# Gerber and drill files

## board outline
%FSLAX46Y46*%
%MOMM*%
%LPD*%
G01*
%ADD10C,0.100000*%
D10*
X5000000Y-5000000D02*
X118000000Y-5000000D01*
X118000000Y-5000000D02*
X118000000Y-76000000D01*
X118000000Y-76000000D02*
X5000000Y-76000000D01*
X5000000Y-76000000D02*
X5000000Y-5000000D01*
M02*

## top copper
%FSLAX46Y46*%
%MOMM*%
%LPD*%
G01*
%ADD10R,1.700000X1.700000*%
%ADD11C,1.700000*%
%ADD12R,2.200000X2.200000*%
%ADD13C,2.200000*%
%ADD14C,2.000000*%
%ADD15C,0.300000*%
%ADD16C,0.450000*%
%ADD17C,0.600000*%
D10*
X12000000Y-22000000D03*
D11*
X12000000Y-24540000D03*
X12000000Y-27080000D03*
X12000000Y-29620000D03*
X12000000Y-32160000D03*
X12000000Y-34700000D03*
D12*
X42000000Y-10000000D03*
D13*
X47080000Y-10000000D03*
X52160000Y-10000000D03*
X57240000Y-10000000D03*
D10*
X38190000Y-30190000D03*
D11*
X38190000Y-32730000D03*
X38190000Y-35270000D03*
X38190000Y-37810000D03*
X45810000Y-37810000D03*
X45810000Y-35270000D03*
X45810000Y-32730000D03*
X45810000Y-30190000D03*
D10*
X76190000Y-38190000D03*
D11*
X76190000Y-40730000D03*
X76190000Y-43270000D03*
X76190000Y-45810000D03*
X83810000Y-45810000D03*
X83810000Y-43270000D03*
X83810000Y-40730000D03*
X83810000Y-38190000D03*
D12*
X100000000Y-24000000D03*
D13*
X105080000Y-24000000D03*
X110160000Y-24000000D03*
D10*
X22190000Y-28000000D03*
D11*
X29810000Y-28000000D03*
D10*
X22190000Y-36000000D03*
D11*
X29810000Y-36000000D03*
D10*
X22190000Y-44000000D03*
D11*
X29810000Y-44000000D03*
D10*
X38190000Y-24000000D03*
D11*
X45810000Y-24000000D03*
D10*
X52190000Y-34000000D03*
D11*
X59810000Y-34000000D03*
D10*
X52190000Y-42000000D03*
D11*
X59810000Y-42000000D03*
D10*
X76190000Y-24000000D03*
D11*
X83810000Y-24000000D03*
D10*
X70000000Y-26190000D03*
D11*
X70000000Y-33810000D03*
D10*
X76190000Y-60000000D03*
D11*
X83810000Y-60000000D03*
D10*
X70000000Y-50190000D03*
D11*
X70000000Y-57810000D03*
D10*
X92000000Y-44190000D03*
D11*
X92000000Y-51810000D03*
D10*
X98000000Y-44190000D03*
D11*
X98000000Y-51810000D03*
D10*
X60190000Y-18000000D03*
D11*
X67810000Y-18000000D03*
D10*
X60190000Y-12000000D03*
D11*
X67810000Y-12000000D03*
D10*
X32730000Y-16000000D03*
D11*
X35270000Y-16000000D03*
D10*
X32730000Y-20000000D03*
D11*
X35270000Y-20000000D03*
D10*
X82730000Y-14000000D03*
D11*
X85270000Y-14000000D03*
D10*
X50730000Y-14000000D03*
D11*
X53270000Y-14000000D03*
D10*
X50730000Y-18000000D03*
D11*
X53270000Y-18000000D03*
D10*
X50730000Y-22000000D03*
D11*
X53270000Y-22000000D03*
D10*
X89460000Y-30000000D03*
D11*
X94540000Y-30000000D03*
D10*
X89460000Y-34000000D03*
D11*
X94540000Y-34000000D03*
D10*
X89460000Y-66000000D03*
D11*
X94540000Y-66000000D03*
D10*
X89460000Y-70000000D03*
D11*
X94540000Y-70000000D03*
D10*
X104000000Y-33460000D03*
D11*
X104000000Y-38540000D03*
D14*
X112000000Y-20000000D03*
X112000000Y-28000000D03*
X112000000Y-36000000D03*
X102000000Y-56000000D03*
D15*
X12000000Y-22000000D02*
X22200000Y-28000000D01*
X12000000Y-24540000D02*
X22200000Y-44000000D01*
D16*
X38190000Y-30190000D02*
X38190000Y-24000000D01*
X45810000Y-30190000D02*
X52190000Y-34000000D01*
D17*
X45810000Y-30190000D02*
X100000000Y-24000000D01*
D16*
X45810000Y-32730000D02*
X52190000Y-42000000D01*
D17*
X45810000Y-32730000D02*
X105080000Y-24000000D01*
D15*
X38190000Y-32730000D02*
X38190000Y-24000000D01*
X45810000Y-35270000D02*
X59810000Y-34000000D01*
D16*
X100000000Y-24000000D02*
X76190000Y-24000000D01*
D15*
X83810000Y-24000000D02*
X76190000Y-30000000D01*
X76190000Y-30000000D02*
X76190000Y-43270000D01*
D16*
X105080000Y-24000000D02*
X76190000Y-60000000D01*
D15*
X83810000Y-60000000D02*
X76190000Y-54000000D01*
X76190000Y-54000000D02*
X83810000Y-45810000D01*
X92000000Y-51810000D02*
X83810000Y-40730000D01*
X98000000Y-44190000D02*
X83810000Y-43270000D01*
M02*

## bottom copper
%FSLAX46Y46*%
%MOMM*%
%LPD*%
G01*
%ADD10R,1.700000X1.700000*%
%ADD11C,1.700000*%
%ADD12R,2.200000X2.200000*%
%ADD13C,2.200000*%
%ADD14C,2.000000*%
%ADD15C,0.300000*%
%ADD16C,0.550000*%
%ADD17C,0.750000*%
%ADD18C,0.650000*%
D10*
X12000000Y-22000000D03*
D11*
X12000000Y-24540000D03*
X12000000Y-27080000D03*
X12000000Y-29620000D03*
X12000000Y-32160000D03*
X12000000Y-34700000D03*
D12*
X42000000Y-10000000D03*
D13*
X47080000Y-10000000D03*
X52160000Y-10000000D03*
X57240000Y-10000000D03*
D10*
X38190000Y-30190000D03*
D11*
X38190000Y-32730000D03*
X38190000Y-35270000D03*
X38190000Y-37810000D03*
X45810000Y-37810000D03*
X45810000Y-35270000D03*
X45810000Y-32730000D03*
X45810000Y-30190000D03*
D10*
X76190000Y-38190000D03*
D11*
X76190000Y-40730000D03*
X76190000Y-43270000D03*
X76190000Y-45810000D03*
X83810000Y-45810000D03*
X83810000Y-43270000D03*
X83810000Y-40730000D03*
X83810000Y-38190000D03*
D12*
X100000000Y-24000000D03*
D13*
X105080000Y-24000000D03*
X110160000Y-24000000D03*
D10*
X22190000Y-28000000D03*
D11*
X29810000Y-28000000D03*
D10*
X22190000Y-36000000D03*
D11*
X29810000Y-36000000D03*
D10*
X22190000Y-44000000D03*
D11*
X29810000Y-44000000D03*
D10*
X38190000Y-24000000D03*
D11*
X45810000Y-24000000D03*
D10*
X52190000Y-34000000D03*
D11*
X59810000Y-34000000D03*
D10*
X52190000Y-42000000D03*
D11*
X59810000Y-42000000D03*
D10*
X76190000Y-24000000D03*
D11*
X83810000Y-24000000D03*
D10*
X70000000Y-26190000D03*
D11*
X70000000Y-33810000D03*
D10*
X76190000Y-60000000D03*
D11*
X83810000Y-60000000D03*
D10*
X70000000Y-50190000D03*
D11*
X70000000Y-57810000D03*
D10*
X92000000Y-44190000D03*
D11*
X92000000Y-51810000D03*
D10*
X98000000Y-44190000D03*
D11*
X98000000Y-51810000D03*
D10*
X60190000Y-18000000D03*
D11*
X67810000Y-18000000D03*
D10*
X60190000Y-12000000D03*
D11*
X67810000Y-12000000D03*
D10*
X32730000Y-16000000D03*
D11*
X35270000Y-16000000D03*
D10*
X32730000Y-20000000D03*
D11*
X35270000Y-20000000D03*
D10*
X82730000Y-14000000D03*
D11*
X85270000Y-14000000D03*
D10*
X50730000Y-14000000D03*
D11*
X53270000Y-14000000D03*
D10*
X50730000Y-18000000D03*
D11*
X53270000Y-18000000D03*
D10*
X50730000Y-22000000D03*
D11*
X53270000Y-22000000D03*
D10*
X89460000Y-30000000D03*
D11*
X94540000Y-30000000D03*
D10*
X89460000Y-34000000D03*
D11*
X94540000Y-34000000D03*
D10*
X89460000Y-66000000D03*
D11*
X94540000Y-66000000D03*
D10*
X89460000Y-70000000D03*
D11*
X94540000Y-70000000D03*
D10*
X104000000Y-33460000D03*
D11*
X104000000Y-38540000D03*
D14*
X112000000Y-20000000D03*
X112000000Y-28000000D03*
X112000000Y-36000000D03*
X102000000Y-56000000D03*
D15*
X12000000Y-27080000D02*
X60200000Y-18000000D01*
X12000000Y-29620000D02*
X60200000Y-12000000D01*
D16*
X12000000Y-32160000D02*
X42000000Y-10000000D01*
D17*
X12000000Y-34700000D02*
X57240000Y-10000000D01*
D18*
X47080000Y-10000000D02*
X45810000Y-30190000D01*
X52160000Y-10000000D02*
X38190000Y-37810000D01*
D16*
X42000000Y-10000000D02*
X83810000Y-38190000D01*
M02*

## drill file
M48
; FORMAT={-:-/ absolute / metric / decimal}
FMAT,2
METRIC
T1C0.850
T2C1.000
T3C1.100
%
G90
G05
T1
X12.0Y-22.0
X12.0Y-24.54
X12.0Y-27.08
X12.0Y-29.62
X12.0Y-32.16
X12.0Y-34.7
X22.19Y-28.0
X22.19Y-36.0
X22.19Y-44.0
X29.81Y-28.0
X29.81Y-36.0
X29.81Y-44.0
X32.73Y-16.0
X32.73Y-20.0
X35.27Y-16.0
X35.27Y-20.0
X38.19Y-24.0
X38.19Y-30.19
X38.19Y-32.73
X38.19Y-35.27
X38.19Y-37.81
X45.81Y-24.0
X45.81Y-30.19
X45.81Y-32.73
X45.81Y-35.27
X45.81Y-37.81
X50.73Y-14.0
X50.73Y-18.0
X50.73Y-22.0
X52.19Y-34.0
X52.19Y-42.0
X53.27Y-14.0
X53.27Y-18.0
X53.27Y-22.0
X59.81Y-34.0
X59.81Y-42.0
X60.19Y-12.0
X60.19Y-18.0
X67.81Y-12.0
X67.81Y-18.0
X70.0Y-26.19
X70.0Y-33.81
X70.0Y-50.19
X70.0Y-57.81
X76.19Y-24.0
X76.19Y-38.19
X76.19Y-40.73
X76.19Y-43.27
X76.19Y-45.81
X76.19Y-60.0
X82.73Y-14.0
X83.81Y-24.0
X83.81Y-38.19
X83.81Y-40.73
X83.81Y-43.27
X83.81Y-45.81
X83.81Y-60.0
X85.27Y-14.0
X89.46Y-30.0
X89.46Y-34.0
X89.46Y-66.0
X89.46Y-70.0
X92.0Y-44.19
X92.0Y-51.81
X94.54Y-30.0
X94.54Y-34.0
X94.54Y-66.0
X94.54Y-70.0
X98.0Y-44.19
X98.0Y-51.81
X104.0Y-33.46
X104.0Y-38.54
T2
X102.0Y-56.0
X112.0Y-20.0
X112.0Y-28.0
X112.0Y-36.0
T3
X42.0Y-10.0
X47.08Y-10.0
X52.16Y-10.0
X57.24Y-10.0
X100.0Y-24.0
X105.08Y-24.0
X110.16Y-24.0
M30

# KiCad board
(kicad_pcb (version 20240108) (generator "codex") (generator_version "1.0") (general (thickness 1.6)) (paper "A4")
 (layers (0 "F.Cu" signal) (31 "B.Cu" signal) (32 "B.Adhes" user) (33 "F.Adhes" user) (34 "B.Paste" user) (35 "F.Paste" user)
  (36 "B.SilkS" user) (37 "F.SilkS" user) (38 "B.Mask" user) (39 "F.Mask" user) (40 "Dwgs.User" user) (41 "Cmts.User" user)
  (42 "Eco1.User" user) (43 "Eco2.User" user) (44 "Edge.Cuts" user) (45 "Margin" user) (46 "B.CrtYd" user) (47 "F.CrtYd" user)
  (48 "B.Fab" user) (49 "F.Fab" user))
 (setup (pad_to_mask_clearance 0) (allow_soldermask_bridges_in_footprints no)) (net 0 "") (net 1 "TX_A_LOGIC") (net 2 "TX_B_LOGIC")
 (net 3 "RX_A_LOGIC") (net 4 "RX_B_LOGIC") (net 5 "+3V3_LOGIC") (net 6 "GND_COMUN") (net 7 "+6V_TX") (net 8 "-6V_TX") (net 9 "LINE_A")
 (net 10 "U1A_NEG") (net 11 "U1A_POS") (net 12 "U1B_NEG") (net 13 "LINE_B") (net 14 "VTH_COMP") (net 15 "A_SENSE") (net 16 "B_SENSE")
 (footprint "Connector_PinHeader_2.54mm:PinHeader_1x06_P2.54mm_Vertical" (layer "F.Cu") (at 12.00 22.00)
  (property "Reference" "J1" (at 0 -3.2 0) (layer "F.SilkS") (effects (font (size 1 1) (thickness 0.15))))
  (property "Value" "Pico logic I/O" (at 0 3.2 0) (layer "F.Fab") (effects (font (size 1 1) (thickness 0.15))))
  (pad "1" thru_hole rect (at 0.00 0.00) (size 1.70 1.70) (drill 0.85) (layers "*.Cu" "*.Mask") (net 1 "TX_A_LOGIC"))
  (pad "2" thru_hole circle (at 0.00 2.54) (size 1.70 1.70) (drill 0.85) (layers "*.Cu" "*.Mask") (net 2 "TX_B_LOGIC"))
  (pad "3" thru_hole circle (at 0.00 5.08) (size 1.70 1.70) (drill 0.85) (layers "*.Cu" "*.Mask") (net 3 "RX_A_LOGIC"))
  (pad "4" thru_hole circle (at 0.00 7.62) (size 1.70 1.70) (drill 0.85) (layers "*.Cu" "*.Mask") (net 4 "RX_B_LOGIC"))
  (pad "5" thru_hole circle (at 0.00 10.16) (size 1.70 1.70) (drill 0.85) (layers "*.Cu" "*.Mask") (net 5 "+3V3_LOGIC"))
  (pad "6" thru_hole circle (at 0.00 12.70) (size 1.70 1.70) (drill 0.85) (layers "*.Cu" "*.Mask") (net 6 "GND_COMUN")))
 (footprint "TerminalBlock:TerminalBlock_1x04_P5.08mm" (layer "F.Cu") (at 42.00 10.00)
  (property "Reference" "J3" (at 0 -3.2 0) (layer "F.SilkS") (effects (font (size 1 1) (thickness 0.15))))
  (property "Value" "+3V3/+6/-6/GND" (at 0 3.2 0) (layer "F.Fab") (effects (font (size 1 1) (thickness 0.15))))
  (pad "1" thru_hole rect (at 0.00 0.00) (size 2.20 2.20) (drill 1.10) (layers "*.Cu" "*.Mask") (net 5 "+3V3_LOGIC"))
  (pad "2" thru_hole circle (at 5.08 0.00) (size 2.20 2.20) (drill 1.10) (layers "*.Cu" "*.Mask") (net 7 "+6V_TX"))
  (pad "3" thru_hole circle (at 10.16 0.00) (size 2.20 2.20) (drill 1.10) (layers "*.Cu" "*.Mask") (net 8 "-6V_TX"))
  (pad "4" thru_hole circle (at 15.24 0.00) (size 2.20 2.20) (drill 1.10) (layers "*.Cu" "*.Mask") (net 6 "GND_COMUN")))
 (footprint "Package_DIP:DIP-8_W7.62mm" (layer "F.Cu") (at 42.00 34.00)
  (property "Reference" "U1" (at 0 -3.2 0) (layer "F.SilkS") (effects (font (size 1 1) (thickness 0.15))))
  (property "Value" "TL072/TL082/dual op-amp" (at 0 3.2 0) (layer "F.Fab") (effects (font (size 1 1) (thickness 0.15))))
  (pad "1" thru_hole rect (at -3.81 -3.81) (size 1.70 1.70) (drill 0.85) (layers "*.Cu" "*.Mask") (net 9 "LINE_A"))
  (pad "2" thru_hole circle (at -3.81 -1.27) (size 1.70 1.70) (drill 0.85) (layers "*.Cu" "*.Mask") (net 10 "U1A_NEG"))
  (pad "3" thru_hole circle (at -3.81 1.27) (size 1.70 1.70) (drill 0.85) (layers "*.Cu" "*.Mask") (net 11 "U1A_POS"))
  (pad "4" thru_hole circle (at -3.81 3.81) (size 1.70 1.70) (drill 0.85) (layers "*.Cu" "*.Mask") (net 8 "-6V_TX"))
  (pad "5" thru_hole circle (at 3.81 3.81) (size 1.70 1.70) (drill 0.85) (layers "*.Cu" "*.Mask") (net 6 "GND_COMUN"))
  (pad "6" thru_hole circle (at 3.81 1.27) (size 1.70 1.70) (drill 0.85) (layers "*.Cu" "*.Mask") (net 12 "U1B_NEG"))
  (pad "7" thru_hole circle (at 3.81 -1.27) (size 1.70 1.70) (drill 0.85) (layers "*.Cu" "*.Mask") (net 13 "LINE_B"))
  (pad "8" thru_hole circle (at 3.81 -3.81) (size 1.70 1.70) (drill 0.85) (layers "*.Cu" "*.Mask") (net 7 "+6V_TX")))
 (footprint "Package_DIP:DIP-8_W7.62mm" (layer "F.Cu") (at 80.00 42.00)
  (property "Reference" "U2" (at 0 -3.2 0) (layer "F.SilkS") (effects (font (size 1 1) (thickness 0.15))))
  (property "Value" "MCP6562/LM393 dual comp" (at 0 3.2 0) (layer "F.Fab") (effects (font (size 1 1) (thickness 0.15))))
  (pad "1" thru_hole rect (at -3.81 -3.81) (size 1.70 1.70) (drill 0.85) (layers "*.Cu" "*.Mask") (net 3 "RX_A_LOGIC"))
  (pad "2" thru_hole circle (at -3.81 -1.27) (size 1.70 1.70) (drill 0.85) (layers "*.Cu" "*.Mask") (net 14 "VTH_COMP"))
  (pad "3" thru_hole circle (at -3.81 1.27) (size 1.70 1.70) (drill 0.85) (layers "*.Cu" "*.Mask") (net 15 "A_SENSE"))
  (pad "4" thru_hole circle (at -3.81 3.81) (size 1.70 1.70) (drill 0.85) (layers "*.Cu" "*.Mask") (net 6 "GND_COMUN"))
  (pad "5" thru_hole circle (at 3.81 3.81) (size 1.70 1.70) (drill 0.85) (layers "*.Cu" "*.Mask") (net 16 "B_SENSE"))
  (pad "6" thru_hole circle (at 3.81 1.27) (size 1.70 1.70) (drill 0.85) (layers "*.Cu" "*.Mask") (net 14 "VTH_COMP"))
  (pad "7" thru_hole circle (at 3.81 -1.27) (size 1.70 1.70) (drill 0.85) (layers "*.Cu" "*.Mask") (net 4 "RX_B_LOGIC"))
  (pad "8" thru_hole circle (at 3.81 -3.81) (size 1.70 1.70) (drill 0.85) (layers "*.Cu" "*.Mask") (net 5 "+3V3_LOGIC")))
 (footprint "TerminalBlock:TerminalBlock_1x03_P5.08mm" (layer "F.Cu") (at 100.00 24.00)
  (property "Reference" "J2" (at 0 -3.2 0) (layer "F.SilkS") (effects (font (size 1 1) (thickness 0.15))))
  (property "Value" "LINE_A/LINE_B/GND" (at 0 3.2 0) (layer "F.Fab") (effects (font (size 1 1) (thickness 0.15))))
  (pad "1" thru_hole rect (at 0.00 0.00) (size 2.20 2.20) (drill 1.10) (layers "*.Cu" "*.Mask") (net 9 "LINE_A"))
  (pad "2" thru_hole circle (at 5.08 0.00) (size 2.20 2.20) (drill 1.10) (layers "*.Cu" "*.Mask") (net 13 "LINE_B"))
  (pad "3" thru_hole circle (at 10.16 0.00) (size 2.20 2.20) (drill 1.10) (layers "*.Cu" "*.Mask") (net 6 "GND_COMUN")))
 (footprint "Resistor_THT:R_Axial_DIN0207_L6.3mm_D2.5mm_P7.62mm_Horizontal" (layer "F.Cu") (at 26.00 28.00)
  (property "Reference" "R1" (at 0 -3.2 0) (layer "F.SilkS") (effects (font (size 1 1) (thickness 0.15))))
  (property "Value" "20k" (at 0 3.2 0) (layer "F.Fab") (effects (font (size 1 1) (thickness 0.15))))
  (pad "1" thru_hole rect (at -3.81 0.00) (size 1.70 1.70) (drill 0.85) (layers "*.Cu" "*.Mask") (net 1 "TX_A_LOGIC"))
  (pad "2" thru_hole circle (at 3.81 0.00) (size 1.70 1.70) (drill 0.85) (layers "*.Cu" "*.Mask") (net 11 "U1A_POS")))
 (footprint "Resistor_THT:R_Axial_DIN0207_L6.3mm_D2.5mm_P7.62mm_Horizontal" (layer "F.Cu") (at 26.00 36.00)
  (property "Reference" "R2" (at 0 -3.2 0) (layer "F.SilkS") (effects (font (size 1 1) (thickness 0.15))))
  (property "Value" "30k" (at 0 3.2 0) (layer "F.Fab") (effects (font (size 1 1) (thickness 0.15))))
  (pad "1" thru_hole rect (at -3.81 0.00) (size 1.70 1.70) (drill 0.85) (layers "*.Cu" "*.Mask") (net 11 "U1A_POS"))
  (pad "2" thru_hole circle (at 3.81 0.00) (size 1.70 1.70) (drill 0.85) (layers "*.Cu" "*.Mask") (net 6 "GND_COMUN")))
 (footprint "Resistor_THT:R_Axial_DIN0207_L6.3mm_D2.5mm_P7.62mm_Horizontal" (layer "F.Cu") (at 26.00 44.00)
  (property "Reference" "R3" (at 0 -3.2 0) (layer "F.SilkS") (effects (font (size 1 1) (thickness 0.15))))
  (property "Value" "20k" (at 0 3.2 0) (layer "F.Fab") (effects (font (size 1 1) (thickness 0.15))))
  (pad "1" thru_hole rect (at -3.81 0.00) (size 1.70 1.70) (drill 0.85) (layers "*.Cu" "*.Mask") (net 2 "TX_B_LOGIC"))
  (pad "2" thru_hole circle (at 3.81 0.00) (size 1.70 1.70) (drill 0.85) (layers "*.Cu" "*.Mask") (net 10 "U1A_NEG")))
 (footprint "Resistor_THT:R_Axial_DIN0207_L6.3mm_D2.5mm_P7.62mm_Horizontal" (layer "F.Cu") (at 42.00 24.00)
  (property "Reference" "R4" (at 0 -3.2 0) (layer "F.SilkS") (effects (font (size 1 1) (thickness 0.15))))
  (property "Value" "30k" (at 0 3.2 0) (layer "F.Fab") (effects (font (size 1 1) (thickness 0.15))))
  (pad "1" thru_hole rect (at -3.81 0.00) (size 1.70 1.70) (drill 0.85) (layers "*.Cu" "*.Mask") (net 9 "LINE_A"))
  (pad "2" thru_hole circle (at 3.81 0.00) (size 1.70 1.70) (drill 0.85) (layers "*.Cu" "*.Mask") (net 10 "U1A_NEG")))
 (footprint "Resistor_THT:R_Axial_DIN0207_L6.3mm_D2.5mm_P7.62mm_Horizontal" (layer "F.Cu") (at 56.00 34.00)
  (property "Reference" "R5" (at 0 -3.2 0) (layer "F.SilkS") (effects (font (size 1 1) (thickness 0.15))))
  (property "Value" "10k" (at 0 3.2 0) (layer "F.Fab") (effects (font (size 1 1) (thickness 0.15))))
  (pad "1" thru_hole rect (at -3.81 0.00) (size 1.70 1.70) (drill 0.85) (layers "*.Cu" "*.Mask") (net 9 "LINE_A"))
  (pad "2" thru_hole circle (at 3.81 0.00) (size 1.70 1.70) (drill 0.85) (layers "*.Cu" "*.Mask") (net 12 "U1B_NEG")))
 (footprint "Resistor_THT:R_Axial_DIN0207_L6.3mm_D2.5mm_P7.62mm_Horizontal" (layer "F.Cu") (at 56.00 42.00)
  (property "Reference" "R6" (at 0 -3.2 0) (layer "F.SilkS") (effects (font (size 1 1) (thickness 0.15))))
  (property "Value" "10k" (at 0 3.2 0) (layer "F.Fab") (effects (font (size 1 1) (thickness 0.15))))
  (pad "1" thru_hole rect (at -3.81 0.00) (size 1.70 1.70) (drill 0.85) (layers "*.Cu" "*.Mask") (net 13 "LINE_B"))
  (pad "2" thru_hole circle (at 3.81 0.00) (size 1.70 1.70) (drill 0.85) (layers "*.Cu" "*.Mask") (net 12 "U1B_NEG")))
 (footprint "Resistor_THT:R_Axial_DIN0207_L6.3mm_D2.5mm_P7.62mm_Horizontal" (layer "F.Cu") (at 80.00 24.00)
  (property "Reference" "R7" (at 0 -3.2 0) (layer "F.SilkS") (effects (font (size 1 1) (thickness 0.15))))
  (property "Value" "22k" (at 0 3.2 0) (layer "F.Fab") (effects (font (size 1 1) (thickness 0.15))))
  (pad "1" thru_hole rect (at -3.81 0.00) (size 1.70 1.70) (drill 0.85) (layers "*.Cu" "*.Mask") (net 9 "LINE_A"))
  (pad "2" thru_hole circle (at 3.81 0.00) (size 1.70 1.70) (drill 0.85) (layers "*.Cu" "*.Mask") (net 15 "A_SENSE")))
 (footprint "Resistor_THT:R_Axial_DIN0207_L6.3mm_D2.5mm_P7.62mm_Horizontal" (layer "F.Cu") (at 70.00 30.00)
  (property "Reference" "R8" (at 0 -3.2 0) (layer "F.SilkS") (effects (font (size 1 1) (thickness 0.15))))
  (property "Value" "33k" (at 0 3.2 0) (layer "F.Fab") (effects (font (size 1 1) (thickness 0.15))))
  (pad "1" thru_hole rect (at 0.00 -3.81) (size 1.70 1.70) (drill 0.85) (layers "*.Cu" "*.Mask") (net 15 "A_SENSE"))
  (pad "2" thru_hole circle (at 0.00 3.81) (size 1.70 1.70) (drill 0.85) (layers "*.Cu" "*.Mask") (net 6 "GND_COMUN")))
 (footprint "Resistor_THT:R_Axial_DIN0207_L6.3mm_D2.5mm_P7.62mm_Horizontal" (layer "F.Cu") (at 80.00 60.00)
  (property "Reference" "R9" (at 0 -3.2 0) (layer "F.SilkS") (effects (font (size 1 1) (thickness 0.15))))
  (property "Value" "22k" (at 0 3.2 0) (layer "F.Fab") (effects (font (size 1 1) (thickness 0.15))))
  (pad "1" thru_hole rect (at -3.81 0.00) (size 1.70 1.70) (drill 0.85) (layers "*.Cu" "*.Mask") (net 13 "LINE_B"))
  (pad "2" thru_hole circle (at 3.81 0.00) (size 1.70 1.70) (drill 0.85) (layers "*.Cu" "*.Mask") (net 16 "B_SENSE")))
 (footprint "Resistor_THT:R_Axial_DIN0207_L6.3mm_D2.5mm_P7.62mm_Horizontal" (layer "F.Cu") (at 70.00 54.00)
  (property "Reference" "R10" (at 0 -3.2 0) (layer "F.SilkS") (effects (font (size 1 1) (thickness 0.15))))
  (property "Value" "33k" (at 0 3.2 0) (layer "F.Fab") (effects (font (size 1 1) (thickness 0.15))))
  (pad "1" thru_hole rect (at 0.00 -3.81) (size 1.70 1.70) (drill 0.85) (layers "*.Cu" "*.Mask") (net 16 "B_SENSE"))
  (pad "2" thru_hole circle (at 0.00 3.81) (size 1.70 1.70) (drill 0.85) (layers "*.Cu" "*.Mask") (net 6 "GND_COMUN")))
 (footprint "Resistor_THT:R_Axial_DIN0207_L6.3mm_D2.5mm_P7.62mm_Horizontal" (layer "F.Cu") (at 92.00 48.00)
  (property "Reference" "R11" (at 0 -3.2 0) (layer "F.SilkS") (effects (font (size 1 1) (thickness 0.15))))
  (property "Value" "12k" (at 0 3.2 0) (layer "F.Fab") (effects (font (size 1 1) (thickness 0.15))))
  (pad "1" thru_hole rect (at 0.00 -3.81) (size 1.70 1.70) (drill 0.85) (layers "*.Cu" "*.Mask") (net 5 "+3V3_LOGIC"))
  (pad "2" thru_hole circle (at 0.00 3.81) (size 1.70 1.70) (drill 0.85) (layers "*.Cu" "*.Mask") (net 14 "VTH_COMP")))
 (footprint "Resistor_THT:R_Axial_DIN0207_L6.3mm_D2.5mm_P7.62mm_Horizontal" (layer "F.Cu") (at 98.00 48.00)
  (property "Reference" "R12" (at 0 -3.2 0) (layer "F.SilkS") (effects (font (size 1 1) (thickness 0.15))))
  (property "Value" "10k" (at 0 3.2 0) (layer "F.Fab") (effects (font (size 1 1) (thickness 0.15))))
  (pad "1" thru_hole rect (at 0.00 -3.81) (size 1.70 1.70) (drill 0.85) (layers "*.Cu" "*.Mask") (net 14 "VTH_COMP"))
  (pad "2" thru_hole circle (at 0.00 3.81) (size 1.70 1.70) (drill 0.85) (layers "*.Cu" "*.Mask") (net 6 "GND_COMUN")))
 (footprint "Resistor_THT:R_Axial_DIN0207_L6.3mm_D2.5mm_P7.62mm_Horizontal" (layer "F.Cu") (at 64.00 18.00)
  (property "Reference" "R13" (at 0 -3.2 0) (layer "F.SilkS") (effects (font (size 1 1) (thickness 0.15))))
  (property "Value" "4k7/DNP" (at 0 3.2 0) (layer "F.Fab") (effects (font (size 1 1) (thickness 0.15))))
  (pad "1" thru_hole rect (at -3.81 0.00) (size 1.70 1.70) (drill 0.85) (layers "*.Cu" "*.Mask") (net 5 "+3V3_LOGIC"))
  (pad "2" thru_hole circle (at 3.81 0.00) (size 1.70 1.70) (drill 0.85) (layers "*.Cu" "*.Mask") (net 3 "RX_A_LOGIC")))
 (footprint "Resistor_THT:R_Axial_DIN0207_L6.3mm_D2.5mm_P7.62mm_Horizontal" (layer "F.Cu") (at 64.00 12.00)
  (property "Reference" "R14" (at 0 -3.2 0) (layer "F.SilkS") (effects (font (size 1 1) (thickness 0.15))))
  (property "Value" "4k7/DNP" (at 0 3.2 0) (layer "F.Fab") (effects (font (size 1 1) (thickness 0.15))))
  (pad "1" thru_hole rect (at -3.81 0.00) (size 1.70 1.70) (drill 0.85) (layers "*.Cu" "*.Mask") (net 5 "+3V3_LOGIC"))
  (pad "2" thru_hole circle (at 3.81 0.00) (size 1.70 1.70) (drill 0.85) (layers "*.Cu" "*.Mask") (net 4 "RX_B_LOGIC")))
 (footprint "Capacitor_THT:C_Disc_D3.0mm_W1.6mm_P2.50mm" (layer "F.Cu") (at 34.00 16.00)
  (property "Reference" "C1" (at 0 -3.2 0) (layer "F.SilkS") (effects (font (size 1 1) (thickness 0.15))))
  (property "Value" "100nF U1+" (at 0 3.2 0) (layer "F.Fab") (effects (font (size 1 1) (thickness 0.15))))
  (pad "1" thru_hole rect (at -1.27 0.00) (size 1.70 1.70) (drill 0.85) (layers "*.Cu" "*.Mask") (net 7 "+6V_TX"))
  (pad "2" thru_hole circle (at 1.27 0.00) (size 1.70 1.70) (drill 0.85) (layers "*.Cu" "*.Mask") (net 6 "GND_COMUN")))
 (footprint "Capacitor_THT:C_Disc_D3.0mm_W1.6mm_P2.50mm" (layer "F.Cu") (at 34.00 20.00)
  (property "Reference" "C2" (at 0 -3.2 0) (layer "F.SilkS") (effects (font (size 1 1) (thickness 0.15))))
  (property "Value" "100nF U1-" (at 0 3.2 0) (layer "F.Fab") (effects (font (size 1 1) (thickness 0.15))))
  (pad "1" thru_hole rect (at -1.27 0.00) (size 1.70 1.70) (drill 0.85) (layers "*.Cu" "*.Mask") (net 8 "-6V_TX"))
  (pad "2" thru_hole circle (at 1.27 0.00) (size 1.70 1.70) (drill 0.85) (layers "*.Cu" "*.Mask") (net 6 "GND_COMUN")))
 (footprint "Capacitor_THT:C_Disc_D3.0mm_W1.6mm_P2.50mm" (layer "F.Cu") (at 84.00 14.00)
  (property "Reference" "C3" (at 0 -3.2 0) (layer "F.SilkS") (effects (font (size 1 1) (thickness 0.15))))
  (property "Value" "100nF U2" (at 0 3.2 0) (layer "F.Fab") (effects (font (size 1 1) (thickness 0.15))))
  (pad "1" thru_hole rect (at -1.27 0.00) (size 1.70 1.70) (drill 0.85) (layers "*.Cu" "*.Mask") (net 5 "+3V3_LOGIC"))
  (pad "2" thru_hole circle (at 1.27 0.00) (size 1.70 1.70) (drill 0.85) (layers "*.Cu" "*.Mask") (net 6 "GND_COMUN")))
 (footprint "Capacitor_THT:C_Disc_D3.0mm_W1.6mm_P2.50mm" (layer "F.Cu") (at 52.00 14.00)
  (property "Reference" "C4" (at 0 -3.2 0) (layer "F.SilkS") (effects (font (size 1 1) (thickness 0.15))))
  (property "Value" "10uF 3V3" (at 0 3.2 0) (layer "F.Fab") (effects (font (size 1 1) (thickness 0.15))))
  (pad "1" thru_hole rect (at -1.27 0.00) (size 1.70 1.70) (drill 0.85) (layers "*.Cu" "*.Mask") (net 5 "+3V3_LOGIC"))
  (pad "2" thru_hole circle (at 1.27 0.00) (size 1.70 1.70) (drill 0.85) (layers "*.Cu" "*.Mask") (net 6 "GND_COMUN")))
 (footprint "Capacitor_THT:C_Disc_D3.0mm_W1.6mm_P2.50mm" (layer "F.Cu") (at 52.00 18.00)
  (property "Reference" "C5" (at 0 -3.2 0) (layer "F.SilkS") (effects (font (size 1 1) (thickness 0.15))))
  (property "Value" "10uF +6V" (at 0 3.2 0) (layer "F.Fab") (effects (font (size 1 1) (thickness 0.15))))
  (pad "1" thru_hole rect (at -1.27 0.00) (size 1.70 1.70) (drill 0.85) (layers "*.Cu" "*.Mask") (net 7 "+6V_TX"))
  (pad "2" thru_hole circle (at 1.27 0.00) (size 1.70 1.70) (drill 0.85) (layers "*.Cu" "*.Mask") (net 6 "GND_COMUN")))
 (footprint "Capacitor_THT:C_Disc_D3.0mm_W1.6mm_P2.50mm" (layer "F.Cu") (at 52.00 22.00)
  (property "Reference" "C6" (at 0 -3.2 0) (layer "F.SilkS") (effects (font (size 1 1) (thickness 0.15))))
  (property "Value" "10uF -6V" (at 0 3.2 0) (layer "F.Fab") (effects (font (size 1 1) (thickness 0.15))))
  (pad "1" thru_hole rect (at -1.27 0.00) (size 1.70 1.70) (drill 0.85) (layers "*.Cu" "*.Mask") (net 8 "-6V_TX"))
  (pad "2" thru_hole circle (at 1.27 0.00) (size 1.70 1.70) (drill 0.85) (layers "*.Cu" "*.Mask") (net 6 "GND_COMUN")))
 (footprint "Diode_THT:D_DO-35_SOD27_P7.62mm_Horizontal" (layer "F.Cu") (at 92.00 30.00)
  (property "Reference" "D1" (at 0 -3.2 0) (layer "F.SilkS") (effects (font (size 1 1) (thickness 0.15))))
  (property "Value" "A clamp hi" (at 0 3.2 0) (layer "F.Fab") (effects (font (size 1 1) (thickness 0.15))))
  (pad "1" thru_hole rect (at -2.54 0.00) (size 1.70 1.70) (drill 0.85) (layers "*.Cu" "*.Mask") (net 15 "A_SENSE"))
  (pad "2" thru_hole circle (at 2.54 0.00) (size 1.70 1.70) (drill 0.85) (layers "*.Cu" "*.Mask") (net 5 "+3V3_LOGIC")))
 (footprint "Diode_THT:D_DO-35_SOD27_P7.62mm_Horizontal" (layer "F.Cu") (at 92.00 34.00)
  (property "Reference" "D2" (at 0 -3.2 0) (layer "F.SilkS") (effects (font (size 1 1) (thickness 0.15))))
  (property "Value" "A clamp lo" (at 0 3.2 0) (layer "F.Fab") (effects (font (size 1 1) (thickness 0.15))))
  (pad "1" thru_hole rect (at -2.54 0.00) (size 1.70 1.70) (drill 0.85) (layers "*.Cu" "*.Mask") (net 6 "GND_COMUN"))
  (pad "2" thru_hole circle (at 2.54 0.00) (size 1.70 1.70) (drill 0.85) (layers "*.Cu" "*.Mask") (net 15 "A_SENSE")))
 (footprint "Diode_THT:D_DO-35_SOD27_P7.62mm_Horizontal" (layer "F.Cu") (at 92.00 66.00)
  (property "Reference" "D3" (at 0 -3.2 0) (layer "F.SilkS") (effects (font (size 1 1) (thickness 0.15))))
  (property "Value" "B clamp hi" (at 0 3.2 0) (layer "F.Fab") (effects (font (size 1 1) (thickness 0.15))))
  (pad "1" thru_hole rect (at -2.54 0.00) (size 1.70 1.70) (drill 0.85) (layers "*.Cu" "*.Mask") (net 16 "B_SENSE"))
  (pad "2" thru_hole circle (at 2.54 0.00) (size 1.70 1.70) (drill 0.85) (layers "*.Cu" "*.Mask") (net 5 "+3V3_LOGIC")))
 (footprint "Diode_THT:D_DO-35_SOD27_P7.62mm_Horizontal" (layer "F.Cu") (at 92.00 70.00)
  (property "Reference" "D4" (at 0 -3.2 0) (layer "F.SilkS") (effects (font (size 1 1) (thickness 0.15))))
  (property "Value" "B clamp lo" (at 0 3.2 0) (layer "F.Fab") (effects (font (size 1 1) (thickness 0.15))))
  (pad "1" thru_hole rect (at -2.54 0.00) (size 1.70 1.70) (drill 0.85) (layers "*.Cu" "*.Mask") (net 6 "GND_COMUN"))
  (pad "2" thru_hole circle (at 2.54 0.00) (size 1.70 1.70) (drill 0.85) (layers "*.Cu" "*.Mask") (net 16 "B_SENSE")))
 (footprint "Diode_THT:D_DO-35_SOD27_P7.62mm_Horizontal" (layer "F.Cu") (at 104.00 36.00)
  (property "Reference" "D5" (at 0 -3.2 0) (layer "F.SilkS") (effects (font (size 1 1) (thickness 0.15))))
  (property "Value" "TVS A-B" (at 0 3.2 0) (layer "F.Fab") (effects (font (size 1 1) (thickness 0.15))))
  (pad "1" thru_hole rect (at 0.00 -2.54) (size 1.70 1.70) (drill 0.85) (layers "*.Cu" "*.Mask") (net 9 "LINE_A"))
  (pad "2" thru_hole circle (at 0.00 2.54) (size 1.70 1.70) (drill 0.85) (layers "*.Cu" "*.Mask") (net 13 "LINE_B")))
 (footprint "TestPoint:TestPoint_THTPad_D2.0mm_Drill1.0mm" (layer "F.Cu") (at 112.00 20.00)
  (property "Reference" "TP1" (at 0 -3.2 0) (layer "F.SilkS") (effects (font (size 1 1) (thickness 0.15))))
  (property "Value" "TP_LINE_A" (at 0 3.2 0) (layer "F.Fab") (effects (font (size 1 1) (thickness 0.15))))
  (pad "1" thru_hole circle (at 0.00 0.00) (size 2.00 2.00) (drill 1.00) (layers "*.Cu" "*.Mask") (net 9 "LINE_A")))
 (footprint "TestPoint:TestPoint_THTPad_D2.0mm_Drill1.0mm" (layer "F.Cu") (at 112.00 28.00)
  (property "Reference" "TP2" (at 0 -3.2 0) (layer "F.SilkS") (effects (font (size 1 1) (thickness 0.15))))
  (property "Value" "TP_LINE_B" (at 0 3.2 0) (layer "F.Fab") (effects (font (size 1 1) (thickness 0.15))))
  (pad "1" thru_hole circle (at 0.00 0.00) (size 2.00 2.00) (drill 1.00) (layers "*.Cu" "*.Mask") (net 13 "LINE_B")))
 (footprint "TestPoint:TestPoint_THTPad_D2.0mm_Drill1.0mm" (layer "F.Cu") (at 112.00 36.00)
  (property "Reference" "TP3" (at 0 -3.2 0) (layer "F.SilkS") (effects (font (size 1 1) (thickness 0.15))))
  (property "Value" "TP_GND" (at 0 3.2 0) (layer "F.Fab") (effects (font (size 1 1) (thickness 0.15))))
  (pad "1" thru_hole circle (at 0.00 0.00) (size 2.00 2.00) (drill 1.00) (layers "*.Cu" "*.Mask") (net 6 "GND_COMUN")))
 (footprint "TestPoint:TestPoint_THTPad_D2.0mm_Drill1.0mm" (layer "F.Cu") (at 102.00 56.00)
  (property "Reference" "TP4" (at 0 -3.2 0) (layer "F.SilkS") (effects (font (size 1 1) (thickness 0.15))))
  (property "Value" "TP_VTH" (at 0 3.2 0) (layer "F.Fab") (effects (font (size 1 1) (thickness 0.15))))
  (pad "1" thru_hole circle (at 0.00 0.00) (size 2.00 2.00) (drill 1.00) (layers "*.Cu" "*.Mask") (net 14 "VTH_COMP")))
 (gr_line (start 5.00 5.00) (end 118.00 5.00) (stroke (width 0.1) (type solid)) (layer "Edge.Cuts"))
 (gr_line (start 118.00 5.00) (end 118.00 76.00) (stroke (width 0.1) (type solid)) (layer "Edge.Cuts"))
 (gr_line (start 118.00 76.00) (end 5.00 76.00) (stroke (width 0.1) (type solid)) (layer "Edge.Cuts"))
 (gr_line (start 5.00 76.00) (end 5.00 5.00) (stroke (width 0.1) (type solid)) (layer "Edge.Cuts"))
 (segment (start 12.00 22.00) (end 22.20 28.00) (width 0.30) (layer "F.Cu") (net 1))
 (segment (start 12.00 24.54) (end 22.20 44.00) (width 0.30) (layer "F.Cu") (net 2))
 (segment (start 12.00 27.08) (end 60.20 18.00) (width 0.30) (layer "B.Cu") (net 3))
 (segment (start 12.00 29.62) (end 60.20 12.00) (width 0.30) (layer "B.Cu") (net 4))
 (segment (start 12.00 32.16) (end 42.00 10.00) (width 0.55) (layer "B.Cu") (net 5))
 (segment (start 12.00 34.70) (end 57.24 10.00) (width 0.75) (layer "B.Cu") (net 6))
 (segment (start 47.08 10.00) (end 45.81 30.19) (width 0.65) (layer "B.Cu") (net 7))
 (segment (start 52.16 10.00) (end 38.19 37.81) (width 0.65) (layer "B.Cu") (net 8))
 (segment (start 42.00 10.00) (end 83.81 38.19) (width 0.55) (layer "B.Cu") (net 5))
 (segment (start 38.19 30.19) (end 38.19 24.00) (width 0.45) (layer "F.Cu") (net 9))
 (segment (start 45.81 30.19) (end 52.19 34.00) (width 0.45) (layer "F.Cu") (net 9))
 (segment (start 45.81 30.19) (end 100.00 24.00) (width 0.60) (layer "F.Cu") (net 9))
 (segment (start 45.81 32.73) (end 52.19 42.00) (width 0.45) (layer "F.Cu") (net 13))
 (segment (start 45.81 32.73) (end 105.08 24.00) (width 0.60) (layer "F.Cu") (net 13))
 (segment (start 38.19 32.73) (end 38.19 24.00) (width 0.30) (layer "F.Cu") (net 10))
 (segment (start 45.81 35.27) (end 59.81 34.00) (width 0.30) (layer "F.Cu") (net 12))
 (segment (start 100.00 24.00) (end 76.19 24.00) (width 0.45) (layer "F.Cu") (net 9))
 (segment (start 83.81 24.00) (end 76.19 30.00) (width 0.30) (layer "F.Cu") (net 15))
 (segment (start 76.19 30.00) (end 76.19 43.27) (width 0.30) (layer "F.Cu") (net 15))
 (segment (start 105.08 24.00) (end 76.19 60.00) (width 0.45) (layer "F.Cu") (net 13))
 (segment (start 83.81 60.00) (end 76.19 54.00) (width 0.30) (layer "F.Cu") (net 16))
 (segment (start 76.19 54.00) (end 83.81 45.81) (width 0.30) (layer "F.Cu") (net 16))
 (segment (start 92.00 51.81) (end 83.81 40.73) (width 0.30) (layer "F.Cu") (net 14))
 (segment (start 98.00 44.19) (end 83.81 43.27) (width 0.30) (layer "F.Cu") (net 14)))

